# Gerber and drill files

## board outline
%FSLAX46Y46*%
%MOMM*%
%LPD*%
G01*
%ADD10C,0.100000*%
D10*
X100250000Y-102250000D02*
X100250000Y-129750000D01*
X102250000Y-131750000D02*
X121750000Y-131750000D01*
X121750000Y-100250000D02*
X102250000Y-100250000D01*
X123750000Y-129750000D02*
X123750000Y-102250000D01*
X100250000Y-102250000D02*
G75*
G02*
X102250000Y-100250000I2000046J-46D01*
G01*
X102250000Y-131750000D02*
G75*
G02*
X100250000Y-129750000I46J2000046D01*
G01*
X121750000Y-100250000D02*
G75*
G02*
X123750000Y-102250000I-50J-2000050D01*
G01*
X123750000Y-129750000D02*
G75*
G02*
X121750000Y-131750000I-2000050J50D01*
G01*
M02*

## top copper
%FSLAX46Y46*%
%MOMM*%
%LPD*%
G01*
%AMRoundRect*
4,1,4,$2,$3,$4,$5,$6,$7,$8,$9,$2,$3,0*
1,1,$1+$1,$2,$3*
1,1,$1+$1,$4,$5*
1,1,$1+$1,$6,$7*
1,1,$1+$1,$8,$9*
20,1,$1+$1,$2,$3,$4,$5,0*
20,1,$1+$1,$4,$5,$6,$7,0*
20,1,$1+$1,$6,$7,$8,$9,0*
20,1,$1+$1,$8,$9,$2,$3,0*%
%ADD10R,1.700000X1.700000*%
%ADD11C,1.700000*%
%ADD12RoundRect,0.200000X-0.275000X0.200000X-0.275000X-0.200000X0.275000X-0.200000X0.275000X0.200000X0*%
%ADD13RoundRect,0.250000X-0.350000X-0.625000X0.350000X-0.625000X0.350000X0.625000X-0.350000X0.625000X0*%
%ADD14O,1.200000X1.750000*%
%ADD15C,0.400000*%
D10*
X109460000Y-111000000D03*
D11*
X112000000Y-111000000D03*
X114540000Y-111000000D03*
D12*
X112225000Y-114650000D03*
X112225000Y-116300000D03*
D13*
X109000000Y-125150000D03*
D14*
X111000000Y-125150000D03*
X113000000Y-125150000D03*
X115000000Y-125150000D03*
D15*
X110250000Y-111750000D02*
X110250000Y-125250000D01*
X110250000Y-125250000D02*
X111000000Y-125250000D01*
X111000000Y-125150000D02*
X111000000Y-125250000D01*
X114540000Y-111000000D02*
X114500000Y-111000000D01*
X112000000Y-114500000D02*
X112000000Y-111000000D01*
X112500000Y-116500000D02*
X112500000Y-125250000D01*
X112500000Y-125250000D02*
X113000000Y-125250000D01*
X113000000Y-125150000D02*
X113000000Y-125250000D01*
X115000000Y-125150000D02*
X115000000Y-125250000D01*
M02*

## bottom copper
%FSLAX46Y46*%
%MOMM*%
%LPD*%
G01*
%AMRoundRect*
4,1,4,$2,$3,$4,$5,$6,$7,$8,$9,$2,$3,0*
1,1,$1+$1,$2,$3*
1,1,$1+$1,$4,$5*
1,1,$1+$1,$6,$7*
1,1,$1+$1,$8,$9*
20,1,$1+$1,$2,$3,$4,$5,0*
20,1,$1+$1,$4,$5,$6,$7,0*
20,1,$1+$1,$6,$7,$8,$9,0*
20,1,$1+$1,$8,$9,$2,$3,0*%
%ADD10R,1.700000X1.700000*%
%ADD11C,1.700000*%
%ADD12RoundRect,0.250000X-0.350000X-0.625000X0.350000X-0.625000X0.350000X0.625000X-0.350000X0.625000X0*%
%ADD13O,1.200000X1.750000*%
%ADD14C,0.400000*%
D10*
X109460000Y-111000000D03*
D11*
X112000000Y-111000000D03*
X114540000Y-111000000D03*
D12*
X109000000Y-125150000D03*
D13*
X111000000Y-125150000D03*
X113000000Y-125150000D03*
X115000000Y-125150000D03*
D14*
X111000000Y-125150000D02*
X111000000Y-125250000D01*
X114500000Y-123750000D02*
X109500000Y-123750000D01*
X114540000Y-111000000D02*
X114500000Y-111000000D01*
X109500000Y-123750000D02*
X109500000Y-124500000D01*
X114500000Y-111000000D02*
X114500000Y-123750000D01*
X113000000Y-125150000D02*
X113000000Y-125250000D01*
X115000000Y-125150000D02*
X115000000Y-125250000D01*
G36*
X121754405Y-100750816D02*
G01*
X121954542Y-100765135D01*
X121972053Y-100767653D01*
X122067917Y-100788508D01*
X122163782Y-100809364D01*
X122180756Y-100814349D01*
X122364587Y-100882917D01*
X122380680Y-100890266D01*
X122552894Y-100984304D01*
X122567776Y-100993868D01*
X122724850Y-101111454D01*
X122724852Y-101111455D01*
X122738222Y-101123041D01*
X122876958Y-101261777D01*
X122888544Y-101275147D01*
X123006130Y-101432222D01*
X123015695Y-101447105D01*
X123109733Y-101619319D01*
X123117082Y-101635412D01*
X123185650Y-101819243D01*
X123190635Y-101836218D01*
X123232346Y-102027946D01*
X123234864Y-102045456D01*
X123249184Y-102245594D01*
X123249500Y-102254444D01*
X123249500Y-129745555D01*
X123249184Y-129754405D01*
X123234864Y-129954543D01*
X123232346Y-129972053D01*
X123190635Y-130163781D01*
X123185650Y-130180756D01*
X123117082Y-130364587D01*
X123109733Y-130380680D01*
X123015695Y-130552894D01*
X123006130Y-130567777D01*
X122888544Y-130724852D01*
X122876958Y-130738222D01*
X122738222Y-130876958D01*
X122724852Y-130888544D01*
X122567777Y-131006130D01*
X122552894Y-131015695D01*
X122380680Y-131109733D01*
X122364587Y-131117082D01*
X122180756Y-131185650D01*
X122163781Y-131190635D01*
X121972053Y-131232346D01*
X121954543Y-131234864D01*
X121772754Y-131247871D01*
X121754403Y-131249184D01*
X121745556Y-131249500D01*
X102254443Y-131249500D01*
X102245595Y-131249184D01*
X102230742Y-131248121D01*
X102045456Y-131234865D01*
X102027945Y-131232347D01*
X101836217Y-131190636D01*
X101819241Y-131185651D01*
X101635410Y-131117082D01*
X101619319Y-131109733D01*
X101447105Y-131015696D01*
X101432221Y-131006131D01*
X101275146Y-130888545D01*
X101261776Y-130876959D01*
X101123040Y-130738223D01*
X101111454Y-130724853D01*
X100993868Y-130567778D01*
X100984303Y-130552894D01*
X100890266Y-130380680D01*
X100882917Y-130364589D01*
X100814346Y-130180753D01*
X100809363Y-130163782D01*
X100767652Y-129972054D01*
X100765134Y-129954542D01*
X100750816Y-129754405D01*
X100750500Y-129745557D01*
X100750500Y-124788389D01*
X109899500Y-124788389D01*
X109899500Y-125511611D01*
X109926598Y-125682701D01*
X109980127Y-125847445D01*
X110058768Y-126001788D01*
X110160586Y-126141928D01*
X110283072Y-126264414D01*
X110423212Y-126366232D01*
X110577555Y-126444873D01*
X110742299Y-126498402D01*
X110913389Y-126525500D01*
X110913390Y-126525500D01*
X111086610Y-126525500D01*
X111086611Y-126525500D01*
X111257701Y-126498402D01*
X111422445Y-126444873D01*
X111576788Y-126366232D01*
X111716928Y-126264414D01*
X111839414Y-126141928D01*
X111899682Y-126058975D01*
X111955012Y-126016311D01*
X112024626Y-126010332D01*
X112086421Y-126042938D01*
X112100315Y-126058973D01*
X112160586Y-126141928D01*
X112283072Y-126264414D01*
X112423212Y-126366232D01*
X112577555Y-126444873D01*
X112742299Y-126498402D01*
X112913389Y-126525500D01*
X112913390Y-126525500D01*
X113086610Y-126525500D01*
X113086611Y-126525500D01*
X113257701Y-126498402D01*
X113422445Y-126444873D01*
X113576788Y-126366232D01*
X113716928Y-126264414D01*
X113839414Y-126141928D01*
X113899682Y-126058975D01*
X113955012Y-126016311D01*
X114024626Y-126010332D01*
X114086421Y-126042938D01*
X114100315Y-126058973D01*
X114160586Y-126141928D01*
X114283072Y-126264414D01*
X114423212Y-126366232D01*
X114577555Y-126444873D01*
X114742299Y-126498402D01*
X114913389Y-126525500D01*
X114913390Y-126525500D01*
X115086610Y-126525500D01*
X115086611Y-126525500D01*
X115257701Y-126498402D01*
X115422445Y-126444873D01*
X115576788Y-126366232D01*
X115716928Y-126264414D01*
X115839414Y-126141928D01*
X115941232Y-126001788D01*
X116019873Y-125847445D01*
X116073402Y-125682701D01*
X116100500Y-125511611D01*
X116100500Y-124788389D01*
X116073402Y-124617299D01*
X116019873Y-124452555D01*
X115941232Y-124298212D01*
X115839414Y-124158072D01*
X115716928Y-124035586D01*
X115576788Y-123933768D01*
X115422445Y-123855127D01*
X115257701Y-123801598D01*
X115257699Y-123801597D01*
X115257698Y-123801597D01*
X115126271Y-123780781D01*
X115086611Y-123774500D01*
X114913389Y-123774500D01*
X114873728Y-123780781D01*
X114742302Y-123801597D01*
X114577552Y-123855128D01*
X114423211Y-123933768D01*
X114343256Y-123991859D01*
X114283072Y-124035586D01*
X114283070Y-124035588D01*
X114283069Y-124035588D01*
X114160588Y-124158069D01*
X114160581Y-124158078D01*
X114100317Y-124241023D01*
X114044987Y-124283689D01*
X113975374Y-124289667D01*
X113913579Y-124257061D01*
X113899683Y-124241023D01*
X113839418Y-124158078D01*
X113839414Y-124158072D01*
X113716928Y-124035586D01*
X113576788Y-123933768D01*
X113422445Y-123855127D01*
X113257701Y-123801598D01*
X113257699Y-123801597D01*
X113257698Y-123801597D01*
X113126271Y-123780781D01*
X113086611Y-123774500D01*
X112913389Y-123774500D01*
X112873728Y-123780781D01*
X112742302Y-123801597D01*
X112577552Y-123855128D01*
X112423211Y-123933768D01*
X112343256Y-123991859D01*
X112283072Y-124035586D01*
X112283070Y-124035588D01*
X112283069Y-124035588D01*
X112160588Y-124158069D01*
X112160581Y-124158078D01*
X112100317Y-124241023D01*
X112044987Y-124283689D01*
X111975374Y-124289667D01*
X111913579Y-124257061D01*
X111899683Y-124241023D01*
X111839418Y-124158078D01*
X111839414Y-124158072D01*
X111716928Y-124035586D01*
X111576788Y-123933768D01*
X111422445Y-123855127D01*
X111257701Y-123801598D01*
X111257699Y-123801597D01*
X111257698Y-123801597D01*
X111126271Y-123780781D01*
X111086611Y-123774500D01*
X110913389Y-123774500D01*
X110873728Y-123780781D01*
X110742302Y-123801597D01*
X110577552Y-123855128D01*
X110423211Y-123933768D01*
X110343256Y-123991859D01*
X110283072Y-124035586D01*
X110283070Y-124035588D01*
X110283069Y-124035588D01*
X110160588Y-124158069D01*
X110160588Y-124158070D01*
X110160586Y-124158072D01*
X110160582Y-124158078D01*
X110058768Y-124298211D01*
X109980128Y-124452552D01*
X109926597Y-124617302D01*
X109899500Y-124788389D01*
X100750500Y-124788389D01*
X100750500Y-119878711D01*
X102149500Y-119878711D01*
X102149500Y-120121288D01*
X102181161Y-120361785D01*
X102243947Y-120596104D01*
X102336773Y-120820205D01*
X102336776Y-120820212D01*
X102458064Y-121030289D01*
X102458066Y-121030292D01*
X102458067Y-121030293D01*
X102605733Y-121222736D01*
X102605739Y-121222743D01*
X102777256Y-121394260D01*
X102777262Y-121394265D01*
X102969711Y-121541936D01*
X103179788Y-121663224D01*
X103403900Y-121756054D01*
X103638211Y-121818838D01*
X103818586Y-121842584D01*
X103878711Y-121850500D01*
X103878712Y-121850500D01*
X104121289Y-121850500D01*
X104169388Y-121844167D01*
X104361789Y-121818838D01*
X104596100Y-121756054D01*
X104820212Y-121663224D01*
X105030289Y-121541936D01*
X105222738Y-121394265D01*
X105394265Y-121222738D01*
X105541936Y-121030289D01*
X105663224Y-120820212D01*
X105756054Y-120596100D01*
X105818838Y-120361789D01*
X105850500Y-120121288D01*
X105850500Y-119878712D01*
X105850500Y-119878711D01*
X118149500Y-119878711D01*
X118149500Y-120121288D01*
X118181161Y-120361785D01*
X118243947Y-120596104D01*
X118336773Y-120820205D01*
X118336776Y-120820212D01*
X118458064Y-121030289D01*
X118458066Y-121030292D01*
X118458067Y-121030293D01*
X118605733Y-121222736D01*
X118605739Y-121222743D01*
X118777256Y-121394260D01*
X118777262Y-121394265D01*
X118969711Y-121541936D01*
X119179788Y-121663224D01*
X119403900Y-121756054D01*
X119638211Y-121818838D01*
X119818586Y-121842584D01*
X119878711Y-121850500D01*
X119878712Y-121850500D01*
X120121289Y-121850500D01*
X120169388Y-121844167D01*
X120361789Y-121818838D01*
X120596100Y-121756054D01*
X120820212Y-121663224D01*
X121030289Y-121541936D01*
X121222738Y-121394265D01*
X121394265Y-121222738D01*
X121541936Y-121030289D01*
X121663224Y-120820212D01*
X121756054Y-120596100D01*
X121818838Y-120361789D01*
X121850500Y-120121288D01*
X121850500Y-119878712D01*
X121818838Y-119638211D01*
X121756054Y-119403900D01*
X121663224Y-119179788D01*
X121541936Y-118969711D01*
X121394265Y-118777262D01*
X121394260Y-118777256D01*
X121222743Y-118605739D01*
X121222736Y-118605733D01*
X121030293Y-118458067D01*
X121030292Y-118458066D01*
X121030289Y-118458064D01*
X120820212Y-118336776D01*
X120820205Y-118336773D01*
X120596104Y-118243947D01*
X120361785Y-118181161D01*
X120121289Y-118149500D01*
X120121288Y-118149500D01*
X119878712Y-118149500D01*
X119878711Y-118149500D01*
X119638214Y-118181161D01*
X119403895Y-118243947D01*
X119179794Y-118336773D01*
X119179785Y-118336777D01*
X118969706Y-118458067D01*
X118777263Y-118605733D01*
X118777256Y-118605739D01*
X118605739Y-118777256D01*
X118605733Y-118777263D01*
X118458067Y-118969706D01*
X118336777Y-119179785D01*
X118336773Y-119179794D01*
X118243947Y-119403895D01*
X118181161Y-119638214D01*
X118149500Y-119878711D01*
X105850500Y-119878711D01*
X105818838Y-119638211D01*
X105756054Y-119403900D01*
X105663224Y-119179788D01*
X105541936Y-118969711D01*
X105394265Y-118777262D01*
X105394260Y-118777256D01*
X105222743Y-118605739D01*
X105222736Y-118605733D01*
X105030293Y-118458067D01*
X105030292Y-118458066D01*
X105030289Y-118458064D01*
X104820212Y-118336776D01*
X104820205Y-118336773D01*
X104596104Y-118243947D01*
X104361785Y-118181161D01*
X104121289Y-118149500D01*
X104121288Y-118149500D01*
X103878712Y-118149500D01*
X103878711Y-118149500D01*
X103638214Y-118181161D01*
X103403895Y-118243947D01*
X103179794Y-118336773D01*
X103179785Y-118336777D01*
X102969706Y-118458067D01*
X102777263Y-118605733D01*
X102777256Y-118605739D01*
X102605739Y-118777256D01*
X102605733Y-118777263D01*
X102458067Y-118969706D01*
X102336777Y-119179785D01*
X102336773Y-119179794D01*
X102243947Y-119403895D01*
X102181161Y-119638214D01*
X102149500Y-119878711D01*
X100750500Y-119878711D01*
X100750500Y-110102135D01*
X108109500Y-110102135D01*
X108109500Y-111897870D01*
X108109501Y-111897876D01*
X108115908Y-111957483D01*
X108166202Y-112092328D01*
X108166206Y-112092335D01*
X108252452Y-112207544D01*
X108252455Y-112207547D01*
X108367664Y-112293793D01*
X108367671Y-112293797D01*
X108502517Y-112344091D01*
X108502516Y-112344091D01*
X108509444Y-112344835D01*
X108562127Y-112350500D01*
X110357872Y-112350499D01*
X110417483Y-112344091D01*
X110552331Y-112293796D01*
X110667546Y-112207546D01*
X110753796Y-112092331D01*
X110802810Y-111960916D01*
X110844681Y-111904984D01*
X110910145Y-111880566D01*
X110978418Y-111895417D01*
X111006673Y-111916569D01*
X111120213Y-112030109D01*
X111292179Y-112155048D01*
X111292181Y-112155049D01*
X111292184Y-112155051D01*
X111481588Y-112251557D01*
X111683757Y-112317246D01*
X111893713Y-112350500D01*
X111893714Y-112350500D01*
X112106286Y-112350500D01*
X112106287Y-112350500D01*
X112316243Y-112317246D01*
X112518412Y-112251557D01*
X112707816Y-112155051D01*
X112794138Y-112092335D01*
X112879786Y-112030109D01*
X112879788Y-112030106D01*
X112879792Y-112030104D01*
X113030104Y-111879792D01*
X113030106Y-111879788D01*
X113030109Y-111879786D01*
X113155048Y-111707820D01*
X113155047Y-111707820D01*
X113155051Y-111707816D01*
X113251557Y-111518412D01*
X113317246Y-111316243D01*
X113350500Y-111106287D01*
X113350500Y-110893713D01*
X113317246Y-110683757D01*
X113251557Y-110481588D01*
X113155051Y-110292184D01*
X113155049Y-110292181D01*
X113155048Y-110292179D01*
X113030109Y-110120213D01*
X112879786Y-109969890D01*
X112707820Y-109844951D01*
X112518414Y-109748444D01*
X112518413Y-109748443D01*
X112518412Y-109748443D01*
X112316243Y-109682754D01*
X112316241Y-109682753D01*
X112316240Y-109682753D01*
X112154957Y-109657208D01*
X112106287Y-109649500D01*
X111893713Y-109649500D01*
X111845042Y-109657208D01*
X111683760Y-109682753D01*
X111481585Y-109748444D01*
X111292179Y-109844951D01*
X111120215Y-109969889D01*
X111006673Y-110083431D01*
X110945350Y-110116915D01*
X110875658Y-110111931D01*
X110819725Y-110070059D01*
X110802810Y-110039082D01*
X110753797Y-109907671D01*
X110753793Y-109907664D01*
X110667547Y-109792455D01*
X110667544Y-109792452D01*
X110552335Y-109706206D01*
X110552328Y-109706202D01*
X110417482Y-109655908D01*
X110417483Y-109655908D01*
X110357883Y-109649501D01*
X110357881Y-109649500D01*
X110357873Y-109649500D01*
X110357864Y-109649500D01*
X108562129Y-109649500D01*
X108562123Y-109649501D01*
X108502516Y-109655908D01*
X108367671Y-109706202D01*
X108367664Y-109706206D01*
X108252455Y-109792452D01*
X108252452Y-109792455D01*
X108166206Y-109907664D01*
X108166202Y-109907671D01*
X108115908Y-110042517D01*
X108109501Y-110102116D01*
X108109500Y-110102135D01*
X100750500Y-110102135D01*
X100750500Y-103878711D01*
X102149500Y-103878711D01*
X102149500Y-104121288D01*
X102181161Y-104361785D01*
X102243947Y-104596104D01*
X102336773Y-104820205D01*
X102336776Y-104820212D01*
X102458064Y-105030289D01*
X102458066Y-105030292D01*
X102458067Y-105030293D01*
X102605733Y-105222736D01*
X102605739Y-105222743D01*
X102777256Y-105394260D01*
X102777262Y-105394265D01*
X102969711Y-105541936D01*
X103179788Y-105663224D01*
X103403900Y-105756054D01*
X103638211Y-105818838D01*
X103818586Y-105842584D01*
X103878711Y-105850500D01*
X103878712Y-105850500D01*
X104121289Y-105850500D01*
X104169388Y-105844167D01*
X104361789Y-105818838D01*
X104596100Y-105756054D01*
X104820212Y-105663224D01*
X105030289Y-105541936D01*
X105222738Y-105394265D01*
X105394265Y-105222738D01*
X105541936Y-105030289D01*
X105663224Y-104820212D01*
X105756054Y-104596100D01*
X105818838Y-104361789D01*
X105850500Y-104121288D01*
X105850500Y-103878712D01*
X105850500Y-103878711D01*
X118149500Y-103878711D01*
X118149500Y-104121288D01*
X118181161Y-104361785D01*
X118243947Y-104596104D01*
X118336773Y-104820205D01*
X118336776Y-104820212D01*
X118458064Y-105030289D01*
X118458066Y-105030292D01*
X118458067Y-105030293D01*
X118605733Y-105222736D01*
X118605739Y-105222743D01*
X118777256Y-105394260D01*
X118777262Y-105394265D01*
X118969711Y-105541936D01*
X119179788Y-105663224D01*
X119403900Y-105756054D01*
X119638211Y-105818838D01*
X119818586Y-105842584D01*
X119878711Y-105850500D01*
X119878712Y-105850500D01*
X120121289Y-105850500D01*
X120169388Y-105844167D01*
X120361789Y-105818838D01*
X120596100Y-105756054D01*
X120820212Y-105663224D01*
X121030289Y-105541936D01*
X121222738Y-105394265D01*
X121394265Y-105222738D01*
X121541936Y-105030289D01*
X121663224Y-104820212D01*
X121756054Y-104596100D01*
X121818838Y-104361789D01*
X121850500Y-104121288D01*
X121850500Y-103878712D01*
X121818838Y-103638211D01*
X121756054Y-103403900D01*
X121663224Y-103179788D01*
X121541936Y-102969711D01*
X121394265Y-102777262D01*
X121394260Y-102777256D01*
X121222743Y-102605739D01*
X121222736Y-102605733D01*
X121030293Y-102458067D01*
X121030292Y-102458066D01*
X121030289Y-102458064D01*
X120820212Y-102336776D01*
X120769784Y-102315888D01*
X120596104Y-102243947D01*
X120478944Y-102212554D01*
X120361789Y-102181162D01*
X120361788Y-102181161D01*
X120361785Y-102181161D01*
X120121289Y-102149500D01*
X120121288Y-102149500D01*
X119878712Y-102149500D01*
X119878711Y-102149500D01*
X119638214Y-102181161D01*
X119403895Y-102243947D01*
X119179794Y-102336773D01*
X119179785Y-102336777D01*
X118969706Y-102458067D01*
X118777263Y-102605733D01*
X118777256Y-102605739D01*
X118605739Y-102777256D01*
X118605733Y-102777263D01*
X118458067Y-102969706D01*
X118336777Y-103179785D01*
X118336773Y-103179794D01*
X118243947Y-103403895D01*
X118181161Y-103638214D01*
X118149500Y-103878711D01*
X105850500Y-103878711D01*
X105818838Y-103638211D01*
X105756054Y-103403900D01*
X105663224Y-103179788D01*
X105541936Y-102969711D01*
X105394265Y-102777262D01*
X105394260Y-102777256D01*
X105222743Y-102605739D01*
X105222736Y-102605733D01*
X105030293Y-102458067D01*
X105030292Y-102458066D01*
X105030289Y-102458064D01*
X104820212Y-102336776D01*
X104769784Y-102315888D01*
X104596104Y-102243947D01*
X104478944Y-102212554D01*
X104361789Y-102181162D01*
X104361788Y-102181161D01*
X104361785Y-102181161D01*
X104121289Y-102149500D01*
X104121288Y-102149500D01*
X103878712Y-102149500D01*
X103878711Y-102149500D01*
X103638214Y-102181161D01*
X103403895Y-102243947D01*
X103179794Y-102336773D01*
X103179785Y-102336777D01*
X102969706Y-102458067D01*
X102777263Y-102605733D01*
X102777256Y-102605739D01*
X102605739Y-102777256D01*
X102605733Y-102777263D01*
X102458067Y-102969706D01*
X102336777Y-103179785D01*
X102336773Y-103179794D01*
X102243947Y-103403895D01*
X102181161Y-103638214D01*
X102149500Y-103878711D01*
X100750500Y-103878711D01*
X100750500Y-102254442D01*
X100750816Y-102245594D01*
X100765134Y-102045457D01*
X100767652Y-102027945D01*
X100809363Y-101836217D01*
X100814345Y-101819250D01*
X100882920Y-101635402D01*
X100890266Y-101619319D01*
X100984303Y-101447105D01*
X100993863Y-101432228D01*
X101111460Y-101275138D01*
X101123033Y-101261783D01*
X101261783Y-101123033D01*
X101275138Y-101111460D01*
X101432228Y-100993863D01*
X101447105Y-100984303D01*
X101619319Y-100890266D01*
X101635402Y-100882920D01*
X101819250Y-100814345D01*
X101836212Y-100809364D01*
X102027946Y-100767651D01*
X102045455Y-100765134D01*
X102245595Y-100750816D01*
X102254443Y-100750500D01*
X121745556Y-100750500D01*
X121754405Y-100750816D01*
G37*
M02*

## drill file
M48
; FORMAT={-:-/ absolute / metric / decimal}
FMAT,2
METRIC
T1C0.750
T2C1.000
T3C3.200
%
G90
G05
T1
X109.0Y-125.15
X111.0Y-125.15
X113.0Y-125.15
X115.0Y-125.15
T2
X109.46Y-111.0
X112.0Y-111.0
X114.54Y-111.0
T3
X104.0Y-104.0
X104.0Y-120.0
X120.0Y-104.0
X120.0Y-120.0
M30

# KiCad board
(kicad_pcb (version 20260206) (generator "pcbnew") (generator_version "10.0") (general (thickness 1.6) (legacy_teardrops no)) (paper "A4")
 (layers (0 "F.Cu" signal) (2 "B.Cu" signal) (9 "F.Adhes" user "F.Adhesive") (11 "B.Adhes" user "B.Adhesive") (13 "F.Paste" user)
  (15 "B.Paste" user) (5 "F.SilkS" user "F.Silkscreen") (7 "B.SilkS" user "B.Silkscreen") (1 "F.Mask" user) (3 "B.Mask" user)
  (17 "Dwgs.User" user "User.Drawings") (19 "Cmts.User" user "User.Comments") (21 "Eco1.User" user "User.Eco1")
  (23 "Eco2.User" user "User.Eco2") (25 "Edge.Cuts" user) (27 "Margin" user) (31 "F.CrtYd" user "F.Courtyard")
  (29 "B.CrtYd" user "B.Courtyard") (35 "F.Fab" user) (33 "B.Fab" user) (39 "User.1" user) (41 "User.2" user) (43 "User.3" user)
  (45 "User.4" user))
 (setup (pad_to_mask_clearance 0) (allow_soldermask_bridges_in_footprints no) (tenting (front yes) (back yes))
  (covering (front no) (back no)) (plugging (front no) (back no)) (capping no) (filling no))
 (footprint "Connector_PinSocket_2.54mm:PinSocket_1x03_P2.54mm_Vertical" (layer "F.Cu") (at 109.46 111 90)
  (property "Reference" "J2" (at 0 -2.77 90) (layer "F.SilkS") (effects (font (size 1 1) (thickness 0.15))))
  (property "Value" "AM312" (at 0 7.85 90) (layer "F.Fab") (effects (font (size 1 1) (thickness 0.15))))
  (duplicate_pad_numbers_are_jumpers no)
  (pad "1" thru_hole rect (at 0 0 90) (size 1.7 1.7) (drill 1) (layers "*.Cu" "*.Mask") (remove_unused_layers no) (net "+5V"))
  (pad "2" thru_hole circle (at 0 2.54 90) (size 1.7 1.7) (drill 1) (layers "*.Cu" "*.Mask") (remove_unused_layers no) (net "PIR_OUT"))
  (pad "3" thru_hole circle (at 0 5.08 90) (size 1.7 1.7) (drill 1) (layers "*.Cu" "*.Mask") (remove_unused_layers no) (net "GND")))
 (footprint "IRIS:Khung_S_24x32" (layer "F.Cu") (at 100 132)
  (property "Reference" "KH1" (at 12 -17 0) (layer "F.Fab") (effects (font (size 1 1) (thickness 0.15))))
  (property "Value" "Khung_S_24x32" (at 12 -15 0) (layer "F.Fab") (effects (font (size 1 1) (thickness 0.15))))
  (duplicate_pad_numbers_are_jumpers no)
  (fp_line (start 0.25 -29.75) (end 0.25 -2.25) (stroke (width 0.1) (type solid)) (layer "Edge.Cuts"))
  (fp_line (start 2.25 -0.25) (end 21.75 -0.25) (stroke (width 0.1) (type solid)) (layer "Edge.Cuts"))
  (fp_line (start 21.75 -31.75) (end 2.25 -31.75) (stroke (width 0.1) (type solid)) (layer "Edge.Cuts"))
  (fp_line (start 23.75 -2.25) (end 23.75 -29.75) (stroke (width 0.1) (type solid)) (layer "Edge.Cuts"))
  (fp_arc (start 0.25 -29.75) (mid 0.8358 -31.1642) (end 2.25 -31.75) (stroke (width 0.1) (type solid)) (layer "Edge.Cuts"))
  (fp_arc (start 2.25 -0.25) (mid 0.8358 -0.8358) (end 0.25 -2.25) (stroke (width 0.1) (type solid)) (layer "Edge.Cuts"))
  (fp_arc (start 21.75 -31.75) (mid 23.164199 -31.164199) (end 23.75 -29.75) (stroke (width 0.1) (type solid)) (layer "Edge.Cuts"))
  (fp_arc (start 23.75 -2.25) (mid 23.164199 -0.835801) (end 21.75 -0.25) (stroke (width 0.1) (type solid)) (layer "Edge.Cuts"))
  (pad "" np_thru_hole circle (at 4 -28) (size 3.2 3.2) (drill 3.2) (layers "*.Cu" "*.Mask"))
  (pad "" np_thru_hole circle (at 4 -12) (size 3.2 3.2) (drill 3.2) (layers "*.Cu" "*.Mask"))
  (pad "" np_thru_hole circle (at 20 -28) (size 3.2 3.2) (drill 3.2) (layers "*.Cu" "*.Mask"))
  (pad "" np_thru_hole circle (at 20 -12) (size 3.2 3.2) (drill 3.2) (layers "*.Cu" "*.Mask")))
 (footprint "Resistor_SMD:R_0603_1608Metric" (layer "F.Cu") (at 112.225 115.475 -90)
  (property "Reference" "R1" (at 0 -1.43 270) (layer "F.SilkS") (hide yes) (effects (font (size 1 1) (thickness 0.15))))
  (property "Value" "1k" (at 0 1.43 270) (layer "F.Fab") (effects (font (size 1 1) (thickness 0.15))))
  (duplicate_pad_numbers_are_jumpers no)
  (pad "1" smd roundrect (at -0.825 0 270) (size 0.8 0.95) (layers "F.Cu" "F.Mask" "F.Paste") (roundrect_rratio 0.25) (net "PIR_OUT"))
  (pad "2" smd roundrect (at 0.825 0 270) (size 0.8 0.95) (layers "F.Cu" "F.Mask" "F.Paste") (roundrect_rratio 0.25) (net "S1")))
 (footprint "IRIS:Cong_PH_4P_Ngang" (layer "F.Cu") (at 109 125.15)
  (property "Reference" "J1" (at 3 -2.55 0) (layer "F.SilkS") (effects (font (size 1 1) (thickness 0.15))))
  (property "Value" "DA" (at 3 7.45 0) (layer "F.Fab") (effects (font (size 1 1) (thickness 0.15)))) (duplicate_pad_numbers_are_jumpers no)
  (pad "1" thru_hole roundrect (at 0 0) (size 1.2 1.75) (drill 0.75) (layers "*.Cu" "*.Mask") (remove_unused_layers no)
   (roundrect_rratio 0.208333) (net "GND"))
  (pad "2" thru_hole oval (at 2 0) (size 1.2 1.75) (drill 0.75) (layers "*.Cu" "*.Mask") (remove_unused_layers no) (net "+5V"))
  (pad "3" thru_hole oval (at 4 0) (size 1.2 1.75) (drill 0.75) (layers "*.Cu" "*.Mask") (remove_unused_layers no) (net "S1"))
  (pad "4" thru_hole oval (at 6 0) (size 1.2 1.75) (drill 0.75) (layers "*.Cu" "*.Mask") (remove_unused_layers no)
   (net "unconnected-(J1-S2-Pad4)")))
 (segment (start 110.25 111.75) (end 110.25 125.25) (width 0.4) (layer "F.Cu") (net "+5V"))
 (segment (start 110.25 125.25) (end 111 125.25) (width 0.4) (layer "F.Cu") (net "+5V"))
 (segment (start 111 125.15) (end 111 125.25) (width 0.4) (layer "F.Cu") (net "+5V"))
 (segment (start 111 125.15) (end 111 125.25) (width 0.4) (layer "B.Cu") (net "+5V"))
 (segment (start 114.54 111) (end 114.5 111) (width 0.4) (layer "F.Cu") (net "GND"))
 (segment (start 114.5 123.75) (end 109.5 123.75) (width 0.4) (layer "B.Cu") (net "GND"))
 (segment (start 114.54 111) (end 114.5 111) (width 0.4) (layer "B.Cu") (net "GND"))
 (segment (start 109.5 123.75) (end 109.5 124.5) (width 0.4) (layer "B.Cu") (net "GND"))
 (segment (start 114.5 111) (end 114.5 123.75) (width 0.4) (layer "B.Cu") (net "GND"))
 (segment (start 112 114.5) (end 112 111) (width 0.4) (layer "F.Cu") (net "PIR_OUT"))
 (segment (start 112.5 116.5) (end 112.5 125.25) (width 0.4) (layer "F.Cu") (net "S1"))
 (segment (start 112.5 125.25) (end 113 125.25) (width 0.4) (layer "F.Cu") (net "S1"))
 (segment (start 113 125.15) (end 113 125.25) (width 0.4) (layer "F.Cu") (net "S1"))
 (segment (start 113 125.15) (end 113 125.25) (width 0.4) (layer "B.Cu") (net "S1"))
 (segment (start 115 125.15) (end 115 125.25) (width 0.4) (layer "F.Cu") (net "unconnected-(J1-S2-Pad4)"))
 (segment (start 115 125.15) (end 115 125.25) (width 0.4) (layer "B.Cu") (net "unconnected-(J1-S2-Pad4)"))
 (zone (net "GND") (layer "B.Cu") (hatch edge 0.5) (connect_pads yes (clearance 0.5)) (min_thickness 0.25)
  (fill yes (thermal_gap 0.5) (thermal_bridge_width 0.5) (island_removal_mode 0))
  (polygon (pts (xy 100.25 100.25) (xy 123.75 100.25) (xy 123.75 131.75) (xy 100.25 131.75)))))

